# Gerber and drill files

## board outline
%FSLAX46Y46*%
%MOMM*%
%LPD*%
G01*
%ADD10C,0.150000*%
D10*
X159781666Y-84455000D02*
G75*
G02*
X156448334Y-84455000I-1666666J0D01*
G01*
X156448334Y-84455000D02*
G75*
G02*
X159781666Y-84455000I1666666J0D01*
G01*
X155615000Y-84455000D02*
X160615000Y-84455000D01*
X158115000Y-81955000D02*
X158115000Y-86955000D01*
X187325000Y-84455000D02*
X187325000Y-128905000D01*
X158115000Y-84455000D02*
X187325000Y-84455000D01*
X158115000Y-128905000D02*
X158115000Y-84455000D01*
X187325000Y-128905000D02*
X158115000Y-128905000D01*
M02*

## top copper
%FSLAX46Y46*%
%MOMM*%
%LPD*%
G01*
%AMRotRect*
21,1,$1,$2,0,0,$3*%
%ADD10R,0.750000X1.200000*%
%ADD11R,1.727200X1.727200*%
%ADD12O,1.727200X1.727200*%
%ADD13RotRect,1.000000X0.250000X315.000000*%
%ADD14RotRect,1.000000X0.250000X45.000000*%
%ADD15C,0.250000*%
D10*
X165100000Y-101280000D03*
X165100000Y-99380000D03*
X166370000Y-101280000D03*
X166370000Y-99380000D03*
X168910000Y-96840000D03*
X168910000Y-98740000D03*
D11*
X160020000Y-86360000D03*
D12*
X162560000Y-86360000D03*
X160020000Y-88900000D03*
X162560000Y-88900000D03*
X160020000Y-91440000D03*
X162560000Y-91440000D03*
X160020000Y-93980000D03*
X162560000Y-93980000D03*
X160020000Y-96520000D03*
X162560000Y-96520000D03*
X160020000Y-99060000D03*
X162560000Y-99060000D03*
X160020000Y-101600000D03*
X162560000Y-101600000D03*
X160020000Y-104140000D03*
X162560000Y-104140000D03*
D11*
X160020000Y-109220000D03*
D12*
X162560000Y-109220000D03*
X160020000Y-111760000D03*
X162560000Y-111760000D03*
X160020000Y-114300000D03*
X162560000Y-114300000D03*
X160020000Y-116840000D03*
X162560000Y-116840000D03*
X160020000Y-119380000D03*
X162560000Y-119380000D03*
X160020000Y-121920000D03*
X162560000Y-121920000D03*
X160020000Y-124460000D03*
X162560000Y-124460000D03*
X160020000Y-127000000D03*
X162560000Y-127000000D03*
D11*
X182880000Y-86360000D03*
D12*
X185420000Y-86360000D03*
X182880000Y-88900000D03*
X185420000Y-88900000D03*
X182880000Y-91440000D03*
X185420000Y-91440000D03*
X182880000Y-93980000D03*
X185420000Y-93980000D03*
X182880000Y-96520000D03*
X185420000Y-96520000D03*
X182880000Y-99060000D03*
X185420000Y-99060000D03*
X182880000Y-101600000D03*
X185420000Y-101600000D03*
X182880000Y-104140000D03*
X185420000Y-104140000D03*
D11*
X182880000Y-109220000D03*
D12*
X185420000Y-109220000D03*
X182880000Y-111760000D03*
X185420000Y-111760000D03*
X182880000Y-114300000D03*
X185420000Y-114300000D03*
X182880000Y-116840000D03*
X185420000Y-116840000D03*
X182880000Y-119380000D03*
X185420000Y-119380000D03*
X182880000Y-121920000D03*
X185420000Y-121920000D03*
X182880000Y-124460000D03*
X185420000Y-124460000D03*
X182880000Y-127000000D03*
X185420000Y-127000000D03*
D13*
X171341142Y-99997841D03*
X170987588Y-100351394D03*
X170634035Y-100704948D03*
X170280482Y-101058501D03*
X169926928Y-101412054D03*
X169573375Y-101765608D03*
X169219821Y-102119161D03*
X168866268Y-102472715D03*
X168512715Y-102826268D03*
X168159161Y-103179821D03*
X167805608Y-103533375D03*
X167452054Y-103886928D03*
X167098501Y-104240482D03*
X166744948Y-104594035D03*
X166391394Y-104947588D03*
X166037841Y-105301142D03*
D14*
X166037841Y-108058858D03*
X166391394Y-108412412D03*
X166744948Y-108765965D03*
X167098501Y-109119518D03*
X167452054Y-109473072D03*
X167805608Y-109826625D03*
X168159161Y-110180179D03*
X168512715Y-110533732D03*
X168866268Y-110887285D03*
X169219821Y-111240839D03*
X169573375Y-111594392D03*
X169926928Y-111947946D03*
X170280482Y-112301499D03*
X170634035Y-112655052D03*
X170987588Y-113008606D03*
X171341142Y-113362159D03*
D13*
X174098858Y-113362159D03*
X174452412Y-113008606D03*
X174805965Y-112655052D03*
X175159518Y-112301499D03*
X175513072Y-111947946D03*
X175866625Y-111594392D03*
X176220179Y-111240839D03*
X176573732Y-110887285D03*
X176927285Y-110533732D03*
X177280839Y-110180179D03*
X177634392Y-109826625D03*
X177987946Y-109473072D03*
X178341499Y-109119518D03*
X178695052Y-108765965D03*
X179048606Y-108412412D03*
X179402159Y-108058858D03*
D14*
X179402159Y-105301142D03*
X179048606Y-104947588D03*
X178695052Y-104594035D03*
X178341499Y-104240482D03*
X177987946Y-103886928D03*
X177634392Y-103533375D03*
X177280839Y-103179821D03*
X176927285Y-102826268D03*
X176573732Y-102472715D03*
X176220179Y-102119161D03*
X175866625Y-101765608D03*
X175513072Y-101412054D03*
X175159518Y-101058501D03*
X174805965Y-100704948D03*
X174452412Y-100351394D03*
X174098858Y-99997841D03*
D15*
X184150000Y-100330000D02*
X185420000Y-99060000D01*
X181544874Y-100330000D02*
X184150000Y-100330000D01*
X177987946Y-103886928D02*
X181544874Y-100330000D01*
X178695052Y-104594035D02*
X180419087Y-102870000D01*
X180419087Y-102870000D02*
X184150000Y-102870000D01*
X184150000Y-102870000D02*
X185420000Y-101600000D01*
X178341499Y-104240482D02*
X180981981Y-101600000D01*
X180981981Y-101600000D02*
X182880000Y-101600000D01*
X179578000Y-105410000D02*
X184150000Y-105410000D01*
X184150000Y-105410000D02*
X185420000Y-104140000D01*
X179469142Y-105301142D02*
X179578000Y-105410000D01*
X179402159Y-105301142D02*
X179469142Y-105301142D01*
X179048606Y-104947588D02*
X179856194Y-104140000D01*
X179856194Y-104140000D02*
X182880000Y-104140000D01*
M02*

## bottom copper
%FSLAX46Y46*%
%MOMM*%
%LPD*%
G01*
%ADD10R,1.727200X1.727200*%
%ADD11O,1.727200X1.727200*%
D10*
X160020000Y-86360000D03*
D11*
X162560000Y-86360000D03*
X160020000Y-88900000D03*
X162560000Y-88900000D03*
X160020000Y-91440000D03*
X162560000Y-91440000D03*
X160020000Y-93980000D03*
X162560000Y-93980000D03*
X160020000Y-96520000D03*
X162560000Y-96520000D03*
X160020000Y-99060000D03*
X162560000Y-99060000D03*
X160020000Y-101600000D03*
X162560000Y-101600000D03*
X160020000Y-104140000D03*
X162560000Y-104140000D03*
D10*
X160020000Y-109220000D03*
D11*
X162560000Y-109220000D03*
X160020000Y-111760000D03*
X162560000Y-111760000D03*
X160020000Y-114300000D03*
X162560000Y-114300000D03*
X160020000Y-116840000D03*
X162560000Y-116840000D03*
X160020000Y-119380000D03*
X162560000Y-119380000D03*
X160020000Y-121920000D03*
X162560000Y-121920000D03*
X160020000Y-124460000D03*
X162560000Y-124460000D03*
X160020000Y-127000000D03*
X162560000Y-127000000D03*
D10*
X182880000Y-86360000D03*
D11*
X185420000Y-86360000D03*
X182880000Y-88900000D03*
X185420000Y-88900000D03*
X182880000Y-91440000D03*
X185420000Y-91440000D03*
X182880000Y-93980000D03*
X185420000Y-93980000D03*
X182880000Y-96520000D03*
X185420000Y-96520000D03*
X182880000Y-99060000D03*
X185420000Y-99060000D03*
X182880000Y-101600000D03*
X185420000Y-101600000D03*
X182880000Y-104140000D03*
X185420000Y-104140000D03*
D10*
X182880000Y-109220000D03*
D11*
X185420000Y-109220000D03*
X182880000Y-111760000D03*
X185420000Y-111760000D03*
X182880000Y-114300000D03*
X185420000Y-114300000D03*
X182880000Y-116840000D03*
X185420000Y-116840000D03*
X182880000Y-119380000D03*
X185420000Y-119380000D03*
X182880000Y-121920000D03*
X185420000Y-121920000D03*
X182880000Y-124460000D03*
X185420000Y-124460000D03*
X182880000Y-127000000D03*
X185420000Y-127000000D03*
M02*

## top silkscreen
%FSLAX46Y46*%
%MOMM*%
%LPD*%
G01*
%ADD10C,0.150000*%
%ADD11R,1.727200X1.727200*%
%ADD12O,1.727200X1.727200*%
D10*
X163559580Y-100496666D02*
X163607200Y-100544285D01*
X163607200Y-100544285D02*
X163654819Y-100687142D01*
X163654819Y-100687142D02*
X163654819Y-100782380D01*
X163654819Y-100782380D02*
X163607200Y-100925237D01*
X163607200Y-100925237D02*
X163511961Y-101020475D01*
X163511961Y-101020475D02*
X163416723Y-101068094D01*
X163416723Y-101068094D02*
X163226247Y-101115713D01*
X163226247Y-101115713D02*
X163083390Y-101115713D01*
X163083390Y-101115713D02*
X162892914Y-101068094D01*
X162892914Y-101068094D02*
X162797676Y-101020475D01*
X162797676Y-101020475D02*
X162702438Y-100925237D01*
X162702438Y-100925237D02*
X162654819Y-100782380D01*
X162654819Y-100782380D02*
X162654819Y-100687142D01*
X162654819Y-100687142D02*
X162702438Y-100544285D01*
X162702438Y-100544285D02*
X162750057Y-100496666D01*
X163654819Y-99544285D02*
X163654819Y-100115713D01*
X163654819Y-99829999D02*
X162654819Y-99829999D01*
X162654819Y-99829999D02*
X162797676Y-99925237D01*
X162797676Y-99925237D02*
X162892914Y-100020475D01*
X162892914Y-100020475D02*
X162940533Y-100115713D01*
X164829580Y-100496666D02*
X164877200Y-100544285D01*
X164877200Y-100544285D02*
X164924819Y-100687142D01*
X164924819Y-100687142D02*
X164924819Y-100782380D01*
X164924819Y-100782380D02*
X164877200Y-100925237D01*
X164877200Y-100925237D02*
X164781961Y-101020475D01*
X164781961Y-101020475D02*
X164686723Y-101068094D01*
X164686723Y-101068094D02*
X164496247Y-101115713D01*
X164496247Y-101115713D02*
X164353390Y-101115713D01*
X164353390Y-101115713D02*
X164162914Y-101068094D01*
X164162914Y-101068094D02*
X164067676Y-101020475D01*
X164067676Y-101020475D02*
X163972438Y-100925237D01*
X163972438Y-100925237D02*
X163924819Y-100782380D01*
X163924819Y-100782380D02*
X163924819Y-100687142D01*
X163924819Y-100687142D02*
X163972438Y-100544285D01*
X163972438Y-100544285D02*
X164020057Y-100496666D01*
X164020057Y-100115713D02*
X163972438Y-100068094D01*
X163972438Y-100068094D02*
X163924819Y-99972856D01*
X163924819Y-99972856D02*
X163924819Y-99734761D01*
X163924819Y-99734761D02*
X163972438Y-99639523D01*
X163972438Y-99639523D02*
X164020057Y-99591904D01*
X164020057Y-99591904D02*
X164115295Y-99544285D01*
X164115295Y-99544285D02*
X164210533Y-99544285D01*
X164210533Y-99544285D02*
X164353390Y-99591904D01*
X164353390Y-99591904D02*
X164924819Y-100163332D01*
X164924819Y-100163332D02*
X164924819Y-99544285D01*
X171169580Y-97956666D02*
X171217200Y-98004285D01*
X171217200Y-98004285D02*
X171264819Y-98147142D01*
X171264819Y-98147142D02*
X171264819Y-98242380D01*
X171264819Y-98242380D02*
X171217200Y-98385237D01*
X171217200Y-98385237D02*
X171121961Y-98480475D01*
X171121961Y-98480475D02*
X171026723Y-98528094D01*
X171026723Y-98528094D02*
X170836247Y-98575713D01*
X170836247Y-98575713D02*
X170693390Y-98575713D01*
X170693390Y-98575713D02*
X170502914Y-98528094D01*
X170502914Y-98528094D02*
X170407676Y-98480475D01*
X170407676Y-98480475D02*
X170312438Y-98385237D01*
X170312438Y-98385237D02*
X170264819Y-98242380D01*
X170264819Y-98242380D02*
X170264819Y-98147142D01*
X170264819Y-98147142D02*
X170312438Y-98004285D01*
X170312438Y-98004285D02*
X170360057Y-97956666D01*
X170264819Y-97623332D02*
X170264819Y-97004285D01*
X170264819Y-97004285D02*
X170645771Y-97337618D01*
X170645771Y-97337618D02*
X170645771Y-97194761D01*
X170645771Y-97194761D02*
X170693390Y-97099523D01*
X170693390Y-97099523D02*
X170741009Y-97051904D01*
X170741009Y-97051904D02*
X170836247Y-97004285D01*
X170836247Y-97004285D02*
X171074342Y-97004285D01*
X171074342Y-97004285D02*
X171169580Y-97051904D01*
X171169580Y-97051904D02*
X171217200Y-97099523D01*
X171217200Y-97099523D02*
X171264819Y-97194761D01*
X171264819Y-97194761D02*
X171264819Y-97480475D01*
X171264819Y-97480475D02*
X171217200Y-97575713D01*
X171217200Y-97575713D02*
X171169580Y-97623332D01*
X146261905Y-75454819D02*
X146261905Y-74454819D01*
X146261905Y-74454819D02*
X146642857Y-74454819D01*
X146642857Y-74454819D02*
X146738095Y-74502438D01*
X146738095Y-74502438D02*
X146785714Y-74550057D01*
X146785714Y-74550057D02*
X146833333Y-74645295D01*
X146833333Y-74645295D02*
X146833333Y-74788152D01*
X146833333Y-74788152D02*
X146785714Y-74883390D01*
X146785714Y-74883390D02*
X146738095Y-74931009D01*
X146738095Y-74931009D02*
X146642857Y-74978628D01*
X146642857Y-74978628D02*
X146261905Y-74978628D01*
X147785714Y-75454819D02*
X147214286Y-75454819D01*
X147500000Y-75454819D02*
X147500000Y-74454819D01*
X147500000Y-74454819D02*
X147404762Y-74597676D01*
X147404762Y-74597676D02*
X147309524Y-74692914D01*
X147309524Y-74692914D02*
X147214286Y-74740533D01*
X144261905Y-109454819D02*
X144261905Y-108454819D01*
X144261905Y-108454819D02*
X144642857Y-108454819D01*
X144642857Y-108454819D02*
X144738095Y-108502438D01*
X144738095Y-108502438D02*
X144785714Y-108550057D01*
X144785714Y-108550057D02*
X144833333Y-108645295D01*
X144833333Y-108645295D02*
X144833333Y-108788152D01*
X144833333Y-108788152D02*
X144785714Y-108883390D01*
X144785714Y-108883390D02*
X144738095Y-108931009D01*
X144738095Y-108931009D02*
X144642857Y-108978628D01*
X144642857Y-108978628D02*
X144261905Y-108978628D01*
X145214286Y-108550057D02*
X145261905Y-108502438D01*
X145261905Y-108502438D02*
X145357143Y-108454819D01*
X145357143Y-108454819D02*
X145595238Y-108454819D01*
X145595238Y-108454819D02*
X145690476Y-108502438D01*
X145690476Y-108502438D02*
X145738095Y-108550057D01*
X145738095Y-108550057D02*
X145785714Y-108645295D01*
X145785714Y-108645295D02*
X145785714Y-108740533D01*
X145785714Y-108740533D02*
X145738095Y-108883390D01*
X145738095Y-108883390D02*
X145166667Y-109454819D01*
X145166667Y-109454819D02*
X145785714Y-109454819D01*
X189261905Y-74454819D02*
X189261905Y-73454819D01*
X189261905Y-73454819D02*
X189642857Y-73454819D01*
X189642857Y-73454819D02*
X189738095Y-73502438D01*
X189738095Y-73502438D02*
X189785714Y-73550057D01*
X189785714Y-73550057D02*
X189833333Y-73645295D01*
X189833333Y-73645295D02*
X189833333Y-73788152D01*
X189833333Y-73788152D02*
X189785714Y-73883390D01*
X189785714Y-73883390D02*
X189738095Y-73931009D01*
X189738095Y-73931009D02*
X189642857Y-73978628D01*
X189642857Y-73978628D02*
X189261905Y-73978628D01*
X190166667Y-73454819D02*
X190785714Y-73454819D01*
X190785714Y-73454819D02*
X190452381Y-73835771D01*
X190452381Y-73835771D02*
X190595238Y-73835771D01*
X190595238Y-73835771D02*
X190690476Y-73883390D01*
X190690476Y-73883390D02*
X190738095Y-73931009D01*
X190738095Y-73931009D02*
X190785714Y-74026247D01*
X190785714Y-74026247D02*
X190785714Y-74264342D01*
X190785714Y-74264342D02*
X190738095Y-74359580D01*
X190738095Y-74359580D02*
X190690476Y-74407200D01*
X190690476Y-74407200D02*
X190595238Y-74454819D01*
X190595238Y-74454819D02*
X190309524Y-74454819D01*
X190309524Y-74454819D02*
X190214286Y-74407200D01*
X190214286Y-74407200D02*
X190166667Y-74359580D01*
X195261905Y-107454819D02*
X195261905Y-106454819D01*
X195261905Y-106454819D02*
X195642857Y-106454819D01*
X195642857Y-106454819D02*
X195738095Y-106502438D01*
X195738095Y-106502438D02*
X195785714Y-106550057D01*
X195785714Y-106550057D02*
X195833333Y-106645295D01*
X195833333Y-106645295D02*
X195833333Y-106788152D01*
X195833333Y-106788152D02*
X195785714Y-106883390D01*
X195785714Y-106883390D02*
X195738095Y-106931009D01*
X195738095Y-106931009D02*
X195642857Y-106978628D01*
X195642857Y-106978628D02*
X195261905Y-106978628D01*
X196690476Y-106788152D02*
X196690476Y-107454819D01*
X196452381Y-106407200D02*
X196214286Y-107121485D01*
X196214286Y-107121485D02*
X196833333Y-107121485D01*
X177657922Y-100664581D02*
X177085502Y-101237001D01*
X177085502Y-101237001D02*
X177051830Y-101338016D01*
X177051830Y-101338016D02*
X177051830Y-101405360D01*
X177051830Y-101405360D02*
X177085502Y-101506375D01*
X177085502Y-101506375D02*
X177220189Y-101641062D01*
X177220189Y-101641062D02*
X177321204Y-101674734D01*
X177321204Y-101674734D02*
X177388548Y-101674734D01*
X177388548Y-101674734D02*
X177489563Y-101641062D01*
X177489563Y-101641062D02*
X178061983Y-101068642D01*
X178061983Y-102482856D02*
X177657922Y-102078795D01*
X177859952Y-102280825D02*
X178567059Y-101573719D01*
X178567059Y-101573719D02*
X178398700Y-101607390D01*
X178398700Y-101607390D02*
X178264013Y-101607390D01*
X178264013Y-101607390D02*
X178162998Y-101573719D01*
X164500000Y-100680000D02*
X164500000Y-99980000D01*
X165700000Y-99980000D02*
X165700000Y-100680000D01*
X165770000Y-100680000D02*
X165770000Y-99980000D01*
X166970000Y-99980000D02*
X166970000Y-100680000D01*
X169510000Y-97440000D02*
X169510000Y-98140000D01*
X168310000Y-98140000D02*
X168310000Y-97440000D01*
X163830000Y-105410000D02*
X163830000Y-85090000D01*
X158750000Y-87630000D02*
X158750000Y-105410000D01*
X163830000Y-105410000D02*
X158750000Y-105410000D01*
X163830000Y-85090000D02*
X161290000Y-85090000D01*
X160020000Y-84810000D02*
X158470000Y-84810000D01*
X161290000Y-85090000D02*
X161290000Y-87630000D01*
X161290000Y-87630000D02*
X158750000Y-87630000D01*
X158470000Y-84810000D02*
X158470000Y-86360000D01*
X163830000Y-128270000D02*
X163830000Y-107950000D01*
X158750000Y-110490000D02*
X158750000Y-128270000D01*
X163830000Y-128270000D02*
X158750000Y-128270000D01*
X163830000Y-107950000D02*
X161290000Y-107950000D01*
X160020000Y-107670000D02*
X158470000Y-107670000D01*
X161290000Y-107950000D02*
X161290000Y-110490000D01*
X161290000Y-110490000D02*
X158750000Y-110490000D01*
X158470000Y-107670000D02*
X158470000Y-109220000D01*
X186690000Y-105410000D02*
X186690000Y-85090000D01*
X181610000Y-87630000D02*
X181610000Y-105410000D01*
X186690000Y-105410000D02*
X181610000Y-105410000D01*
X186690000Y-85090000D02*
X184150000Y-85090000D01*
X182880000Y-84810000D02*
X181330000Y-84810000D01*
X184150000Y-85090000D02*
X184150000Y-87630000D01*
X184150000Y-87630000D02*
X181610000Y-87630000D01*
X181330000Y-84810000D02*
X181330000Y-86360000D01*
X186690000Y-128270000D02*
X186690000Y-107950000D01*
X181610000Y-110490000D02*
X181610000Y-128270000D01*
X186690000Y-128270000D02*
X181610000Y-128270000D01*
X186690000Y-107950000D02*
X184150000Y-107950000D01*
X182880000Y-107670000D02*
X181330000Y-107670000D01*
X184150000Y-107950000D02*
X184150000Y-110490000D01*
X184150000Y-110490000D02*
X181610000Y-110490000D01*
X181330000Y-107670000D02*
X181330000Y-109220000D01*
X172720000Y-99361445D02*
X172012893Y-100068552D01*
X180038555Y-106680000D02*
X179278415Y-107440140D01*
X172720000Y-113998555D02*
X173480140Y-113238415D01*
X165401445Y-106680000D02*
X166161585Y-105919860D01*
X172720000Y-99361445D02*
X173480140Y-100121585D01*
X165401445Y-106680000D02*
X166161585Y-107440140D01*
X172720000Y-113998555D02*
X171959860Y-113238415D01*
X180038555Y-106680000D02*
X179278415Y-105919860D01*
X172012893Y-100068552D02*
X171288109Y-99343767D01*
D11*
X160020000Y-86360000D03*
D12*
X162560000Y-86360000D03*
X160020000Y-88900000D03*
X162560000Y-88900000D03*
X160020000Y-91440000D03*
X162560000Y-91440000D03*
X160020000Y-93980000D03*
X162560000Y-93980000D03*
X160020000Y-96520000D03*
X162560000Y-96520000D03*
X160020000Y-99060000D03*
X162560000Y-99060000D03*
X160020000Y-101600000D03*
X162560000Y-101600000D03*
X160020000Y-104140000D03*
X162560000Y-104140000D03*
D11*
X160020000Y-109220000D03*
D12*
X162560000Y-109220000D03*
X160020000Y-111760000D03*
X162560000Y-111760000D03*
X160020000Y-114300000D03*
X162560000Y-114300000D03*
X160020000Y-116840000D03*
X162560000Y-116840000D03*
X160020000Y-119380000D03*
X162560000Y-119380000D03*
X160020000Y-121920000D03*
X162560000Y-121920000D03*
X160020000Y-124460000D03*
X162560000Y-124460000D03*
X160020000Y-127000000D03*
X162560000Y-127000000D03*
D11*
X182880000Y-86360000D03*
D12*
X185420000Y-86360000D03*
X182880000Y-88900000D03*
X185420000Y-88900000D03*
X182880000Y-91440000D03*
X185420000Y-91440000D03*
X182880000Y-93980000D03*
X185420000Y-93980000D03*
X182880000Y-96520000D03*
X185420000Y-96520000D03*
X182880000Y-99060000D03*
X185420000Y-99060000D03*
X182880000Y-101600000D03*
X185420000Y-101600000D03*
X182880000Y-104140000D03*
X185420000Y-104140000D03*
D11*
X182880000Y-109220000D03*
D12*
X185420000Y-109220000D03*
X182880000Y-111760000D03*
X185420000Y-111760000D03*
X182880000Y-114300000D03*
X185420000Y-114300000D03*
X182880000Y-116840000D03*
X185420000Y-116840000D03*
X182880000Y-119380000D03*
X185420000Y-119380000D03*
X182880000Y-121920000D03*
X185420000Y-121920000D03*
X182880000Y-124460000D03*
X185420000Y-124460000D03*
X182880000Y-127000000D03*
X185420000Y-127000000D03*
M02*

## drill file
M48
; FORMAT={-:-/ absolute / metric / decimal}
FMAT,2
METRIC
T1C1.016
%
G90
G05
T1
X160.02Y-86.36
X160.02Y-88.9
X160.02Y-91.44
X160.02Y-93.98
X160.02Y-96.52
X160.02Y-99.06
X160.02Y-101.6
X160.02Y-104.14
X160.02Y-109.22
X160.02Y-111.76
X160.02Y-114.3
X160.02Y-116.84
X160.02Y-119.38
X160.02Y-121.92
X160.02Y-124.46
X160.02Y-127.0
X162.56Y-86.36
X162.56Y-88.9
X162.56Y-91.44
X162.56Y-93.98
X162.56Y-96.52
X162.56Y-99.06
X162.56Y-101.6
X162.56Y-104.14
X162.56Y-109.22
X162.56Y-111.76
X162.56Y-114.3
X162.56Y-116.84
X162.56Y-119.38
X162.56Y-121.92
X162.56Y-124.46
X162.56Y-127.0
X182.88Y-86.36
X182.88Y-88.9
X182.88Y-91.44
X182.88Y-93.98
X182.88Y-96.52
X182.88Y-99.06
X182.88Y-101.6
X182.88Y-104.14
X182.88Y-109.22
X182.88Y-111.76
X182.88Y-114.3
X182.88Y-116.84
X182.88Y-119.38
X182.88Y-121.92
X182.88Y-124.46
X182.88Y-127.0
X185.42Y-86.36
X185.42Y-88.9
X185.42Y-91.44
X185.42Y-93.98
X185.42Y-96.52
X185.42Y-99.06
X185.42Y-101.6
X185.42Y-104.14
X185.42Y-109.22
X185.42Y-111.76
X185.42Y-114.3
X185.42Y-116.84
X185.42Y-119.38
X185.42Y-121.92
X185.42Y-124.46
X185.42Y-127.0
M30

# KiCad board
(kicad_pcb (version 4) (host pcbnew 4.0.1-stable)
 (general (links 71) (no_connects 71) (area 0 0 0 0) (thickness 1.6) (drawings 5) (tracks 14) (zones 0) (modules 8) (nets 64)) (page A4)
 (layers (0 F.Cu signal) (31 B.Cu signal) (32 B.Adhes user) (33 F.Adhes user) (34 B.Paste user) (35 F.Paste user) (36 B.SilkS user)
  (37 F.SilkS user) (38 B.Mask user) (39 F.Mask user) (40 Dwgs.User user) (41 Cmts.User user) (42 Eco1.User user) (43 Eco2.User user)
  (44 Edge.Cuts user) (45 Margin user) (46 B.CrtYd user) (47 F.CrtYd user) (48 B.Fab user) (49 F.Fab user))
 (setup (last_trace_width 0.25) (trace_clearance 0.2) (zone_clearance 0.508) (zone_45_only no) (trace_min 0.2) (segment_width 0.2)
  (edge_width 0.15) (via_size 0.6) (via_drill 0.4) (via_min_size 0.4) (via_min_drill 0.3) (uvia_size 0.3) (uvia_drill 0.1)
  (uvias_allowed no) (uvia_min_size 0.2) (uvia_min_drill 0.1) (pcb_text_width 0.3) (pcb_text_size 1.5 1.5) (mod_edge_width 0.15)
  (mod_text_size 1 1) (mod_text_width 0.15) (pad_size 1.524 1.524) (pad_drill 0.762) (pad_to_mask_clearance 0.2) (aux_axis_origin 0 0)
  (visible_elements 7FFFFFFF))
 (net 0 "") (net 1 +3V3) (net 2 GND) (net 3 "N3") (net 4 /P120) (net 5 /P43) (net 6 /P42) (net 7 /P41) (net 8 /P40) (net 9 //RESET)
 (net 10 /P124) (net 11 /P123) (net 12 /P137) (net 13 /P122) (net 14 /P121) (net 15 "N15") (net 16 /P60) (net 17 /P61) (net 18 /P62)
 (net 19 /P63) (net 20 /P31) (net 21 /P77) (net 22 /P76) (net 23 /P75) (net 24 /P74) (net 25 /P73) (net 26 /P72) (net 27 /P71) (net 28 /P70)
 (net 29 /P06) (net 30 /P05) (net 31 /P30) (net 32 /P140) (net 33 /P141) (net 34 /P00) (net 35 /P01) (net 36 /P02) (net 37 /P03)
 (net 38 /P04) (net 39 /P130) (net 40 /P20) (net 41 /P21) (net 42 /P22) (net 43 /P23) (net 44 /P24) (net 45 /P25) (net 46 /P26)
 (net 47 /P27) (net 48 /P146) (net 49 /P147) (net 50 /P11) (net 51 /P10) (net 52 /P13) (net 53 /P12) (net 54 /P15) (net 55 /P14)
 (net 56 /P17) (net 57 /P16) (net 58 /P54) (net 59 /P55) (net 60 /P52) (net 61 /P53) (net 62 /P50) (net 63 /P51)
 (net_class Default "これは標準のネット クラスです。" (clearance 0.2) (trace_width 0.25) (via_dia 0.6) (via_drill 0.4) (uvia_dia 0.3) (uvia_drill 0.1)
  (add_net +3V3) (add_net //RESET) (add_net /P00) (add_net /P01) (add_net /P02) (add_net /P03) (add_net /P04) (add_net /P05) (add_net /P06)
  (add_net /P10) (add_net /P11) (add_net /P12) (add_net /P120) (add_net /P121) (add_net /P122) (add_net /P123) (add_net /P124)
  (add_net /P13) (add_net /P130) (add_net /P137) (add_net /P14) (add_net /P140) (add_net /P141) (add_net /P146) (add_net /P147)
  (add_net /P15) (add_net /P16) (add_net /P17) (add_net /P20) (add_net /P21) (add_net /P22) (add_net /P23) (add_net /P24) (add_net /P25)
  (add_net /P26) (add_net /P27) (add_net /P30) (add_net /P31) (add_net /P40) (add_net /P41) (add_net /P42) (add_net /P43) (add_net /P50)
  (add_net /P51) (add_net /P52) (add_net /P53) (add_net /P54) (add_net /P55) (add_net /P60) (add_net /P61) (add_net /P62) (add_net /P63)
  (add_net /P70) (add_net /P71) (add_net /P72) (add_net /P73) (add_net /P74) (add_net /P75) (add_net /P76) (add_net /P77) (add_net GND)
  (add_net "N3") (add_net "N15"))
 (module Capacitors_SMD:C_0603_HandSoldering (layer F.Cu) (at 165.1 100.33 90)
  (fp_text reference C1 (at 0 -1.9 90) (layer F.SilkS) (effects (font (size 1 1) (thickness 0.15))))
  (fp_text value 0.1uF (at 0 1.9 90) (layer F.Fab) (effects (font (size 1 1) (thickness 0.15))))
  (fp_line (start -0.35 -0.6) (end 0.35 -0.6) (layer F.SilkS) (width 0.15))
  (fp_line (start 0.35 0.6) (end -0.35 0.6) (layer F.SilkS) (width 0.15))
  (pad 1 smd rect (at -0.95 0 90) (size 1.2 0.75) (layers F.Cu F.Paste F.Mask) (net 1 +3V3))
  (pad 2 smd rect (at 0.95 0 90) (size 1.2 0.75) (layers F.Cu F.Paste F.Mask) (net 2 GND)))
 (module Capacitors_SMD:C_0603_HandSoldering (layer F.Cu) (at 166.37 100.33 90)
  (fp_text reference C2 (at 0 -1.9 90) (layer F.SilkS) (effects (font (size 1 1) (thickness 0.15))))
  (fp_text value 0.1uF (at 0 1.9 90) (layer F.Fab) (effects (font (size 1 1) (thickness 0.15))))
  (fp_line (start -0.35 -0.6) (end 0.35 -0.6) (layer F.SilkS) (width 0.15))
  (fp_line (start 0.35 0.6) (end -0.35 0.6) (layer F.SilkS) (width 0.15))
  (pad 1 smd rect (at -0.95 0 90) (size 1.2 0.75) (layers F.Cu F.Paste F.Mask) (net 1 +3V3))
  (pad 2 smd rect (at 0.95 0 90) (size 1.2 0.75) (layers F.Cu F.Paste F.Mask) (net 2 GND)))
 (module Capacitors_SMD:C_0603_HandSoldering (layer F.Cu) (at 168.91 97.79 270)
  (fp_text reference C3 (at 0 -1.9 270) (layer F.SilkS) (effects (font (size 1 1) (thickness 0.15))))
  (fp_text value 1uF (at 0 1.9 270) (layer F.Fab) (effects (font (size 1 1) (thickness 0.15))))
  (fp_line (start -0.35 -0.6) (end 0.35 -0.6) (layer F.SilkS) (width 0.15))
  (fp_line (start 0.35 0.6) (end -0.35 0.6) (layer F.SilkS) (width 0.15))
  (pad 1 smd rect (at -0.95 0 270) (size 1.2 0.75) (layers F.Cu F.Paste F.Mask) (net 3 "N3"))
  (pad 2 smd rect (at 0.95 0 270) (size 1.2 0.75) (layers F.Cu F.Paste F.Mask) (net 2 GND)))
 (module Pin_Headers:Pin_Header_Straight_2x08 (layer F.Cu) (at 160.02 86.36)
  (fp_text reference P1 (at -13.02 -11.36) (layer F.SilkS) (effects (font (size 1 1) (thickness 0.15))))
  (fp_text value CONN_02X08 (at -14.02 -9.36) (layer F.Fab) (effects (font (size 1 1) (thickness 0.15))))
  (fp_line (start 3.81 19.05) (end 3.81 -1.27) (layer F.SilkS) (width 0.15))
  (fp_line (start -1.27 1.27) (end -1.27 19.05) (layer F.SilkS) (width 0.15))
  (fp_line (start 3.81 19.05) (end -1.27 19.05) (layer F.SilkS) (width 0.15))
  (fp_line (start 3.81 -1.27) (end 1.27 -1.27) (layer F.SilkS) (width 0.15))
  (fp_line (start 0 -1.55) (end -1.55 -1.55) (layer F.SilkS) (width 0.15))
  (fp_line (start 1.27 -1.27) (end 1.27 1.27) (layer F.SilkS) (width 0.15))
  (fp_line (start 1.27 1.27) (end -1.27 1.27) (layer F.SilkS) (width 0.15))
  (fp_line (start -1.55 -1.55) (end -1.55 0) (layer F.SilkS) (width 0.15))
  (pad 1 thru_hole rect (at 0 0) (size 1.7272 1.7272) (drill 1.016) (layers *.Cu *.Mask F.SilkS) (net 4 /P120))
  (pad 2 thru_hole oval (at 2.54 0) (size 1.7272 1.7272) (drill 1.016) (layers *.Cu *.Mask F.SilkS) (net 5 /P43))
  (pad 3 thru_hole oval (at 0 2.54) (size 1.7272 1.7272) (drill 1.016) (layers *.Cu *.Mask F.SilkS) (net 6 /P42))
  (pad 4 thru_hole oval (at 2.54 2.54) (size 1.7272 1.7272) (drill 1.016) (layers *.Cu *.Mask F.SilkS) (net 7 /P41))
  (pad 5 thru_hole oval (at 0 5.08) (size 1.7272 1.7272) (drill 1.016) (layers *.Cu *.Mask F.SilkS) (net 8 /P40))
  (pad 6 thru_hole oval (at 2.54 5.08) (size 1.7272 1.7272) (drill 1.016) (layers *.Cu *.Mask F.SilkS) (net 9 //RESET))
  (pad 7 thru_hole oval (at 0 7.62) (size 1.7272 1.7272) (drill 1.016) (layers *.Cu *.Mask F.SilkS) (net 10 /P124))
  (pad 8 thru_hole oval (at 2.54 7.62) (size 1.7272 1.7272) (drill 1.016) (layers *.Cu *.Mask F.SilkS) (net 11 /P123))
  (pad 9 thru_hole oval (at 0 10.16) (size 1.7272 1.7272) (drill 1.016) (layers *.Cu *.Mask F.SilkS) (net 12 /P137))
  (pad 10 thru_hole oval (at 2.54 10.16) (size 1.7272 1.7272) (drill 1.016) (layers *.Cu *.Mask F.SilkS) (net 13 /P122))
  (pad 11 thru_hole oval (at 0 12.7) (size 1.7272 1.7272) (drill 1.016) (layers *.Cu *.Mask F.SilkS) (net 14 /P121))
  (pad 12 thru_hole oval (at 2.54 12.7) (size 1.7272 1.7272) (drill 1.016) (layers *.Cu *.Mask F.SilkS) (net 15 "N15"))
  (pad 13 thru_hole oval (at 0 15.24) (size 1.7272 1.7272) (drill 1.016) (layers *.Cu *.Mask F.SilkS) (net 2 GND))
  (pad 14 thru_hole oval (at 2.54 15.24) (size 1.7272 1.7272) (drill 1.016) (layers *.Cu *.Mask F.SilkS) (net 2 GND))
  (pad 15 thru_hole oval (at 0 17.78) (size 1.7272 1.7272) (drill 1.016) (layers *.Cu *.Mask F.SilkS) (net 1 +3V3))
  (pad 16 thru_hole oval (at 2.54 17.78) (size 1.7272 1.7272) (drill 1.016) (layers *.Cu *.Mask F.SilkS) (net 1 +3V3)))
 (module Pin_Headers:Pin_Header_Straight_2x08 (layer F.Cu) (at 160.02 109.22)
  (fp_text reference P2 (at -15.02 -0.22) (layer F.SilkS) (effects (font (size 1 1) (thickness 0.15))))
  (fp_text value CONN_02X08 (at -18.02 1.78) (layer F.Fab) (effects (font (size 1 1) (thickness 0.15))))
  (fp_line (start 3.81 19.05) (end 3.81 -1.27) (layer F.SilkS) (width 0.15))
  (fp_line (start -1.27 1.27) (end -1.27 19.05) (layer F.SilkS) (width 0.15))
  (fp_line (start 3.81 19.05) (end -1.27 19.05) (layer F.SilkS) (width 0.15))
  (fp_line (start 3.81 -1.27) (end 1.27 -1.27) (layer F.SilkS) (width 0.15))
  (fp_line (start 0 -1.55) (end -1.55 -1.55) (layer F.SilkS) (width 0.15))
  (fp_line (start 1.27 -1.27) (end 1.27 1.27) (layer F.SilkS) (width 0.15))
  (fp_line (start 1.27 1.27) (end -1.27 1.27) (layer F.SilkS) (width 0.15))
  (fp_line (start -1.55 -1.55) (end -1.55 0) (layer F.SilkS) (width 0.15))
  (pad 1 thru_hole rect (at 0 0) (size 1.7272 1.7272) (drill 1.016) (layers *.Cu *.Mask F.SilkS) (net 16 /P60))
  (pad 2 thru_hole oval (at 2.54 0) (size 1.7272 1.7272) (drill 1.016) (layers *.Cu *.Mask F.SilkS) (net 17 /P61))
  (pad 3 thru_hole oval (at 0 2.54) (size 1.7272 1.7272) (drill 1.016) (layers *.Cu *.Mask F.SilkS) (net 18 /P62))
  (pad 4 thru_hole oval (at 2.54 2.54) (size 1.7272 1.7272) (drill 1.016) (layers *.Cu *.Mask F.SilkS) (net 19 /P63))
  (pad 5 thru_hole oval (at 0 5.08) (size 1.7272 1.7272) (drill 1.016) (layers *.Cu *.Mask F.SilkS) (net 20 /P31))
  (pad 6 thru_hole oval (at 2.54 5.08) (size 1.7272 1.7272) (drill 1.016) (layers *.Cu *.Mask F.SilkS) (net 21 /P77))
  (pad 7 thru_hole oval (at 0 7.62) (size 1.7272 1.7272) (drill 1.016) (layers *.Cu *.Mask F.SilkS) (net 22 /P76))
  (pad 8 thru_hole oval (at 2.54 7.62) (size 1.7272 1.7272) (drill 1.016) (layers *.Cu *.Mask F.SilkS) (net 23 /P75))
  (pad 9 thru_hole oval (at 0 10.16) (size 1.7272 1.7272) (drill 1.016) (layers *.Cu *.Mask F.SilkS) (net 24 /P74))
  (pad 10 thru_hole oval (at 2.54 10.16) (size 1.7272 1.7272) (drill 1.016) (layers *.Cu *.Mask F.SilkS) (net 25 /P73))
  (pad 11 thru_hole oval (at 0 12.7) (size 1.7272 1.7272) (drill 1.016) (layers *.Cu *.Mask F.SilkS) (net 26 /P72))
  (pad 12 thru_hole oval (at 2.54 12.7) (size 1.7272 1.7272) (drill 1.016) (layers *.Cu *.Mask F.SilkS) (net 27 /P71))
  (pad 13 thru_hole oval (at 0 15.24) (size 1.7272 1.7272) (drill 1.016) (layers *.Cu *.Mask F.SilkS) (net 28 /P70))
  (pad 14 thru_hole oval (at 2.54 15.24) (size 1.7272 1.7272) (drill 1.016) (layers *.Cu *.Mask F.SilkS) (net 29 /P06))
  (pad 15 thru_hole oval (at 0 17.78) (size 1.7272 1.7272) (drill 1.016) (layers *.Cu *.Mask F.SilkS) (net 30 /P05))
  (pad 16 thru_hole oval (at 2.54 17.78) (size 1.7272 1.7272) (drill 1.016) (layers *.Cu *.Mask F.SilkS) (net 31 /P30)))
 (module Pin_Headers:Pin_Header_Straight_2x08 (layer F.Cu) (at 182.88 86.36)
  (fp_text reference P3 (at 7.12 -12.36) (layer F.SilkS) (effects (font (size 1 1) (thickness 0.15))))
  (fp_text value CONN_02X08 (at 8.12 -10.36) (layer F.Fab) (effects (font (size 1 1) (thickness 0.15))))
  (fp_line (start 3.81 19.05) (end 3.81 -1.27) (layer F.SilkS) (width 0.15))
  (fp_line (start -1.27 1.27) (end -1.27 19.05) (layer F.SilkS) (width 0.15))
  (fp_line (start 3.81 19.05) (end -1.27 19.05) (layer F.SilkS) (width 0.15))
  (fp_line (start 3.81 -1.27) (end 1.27 -1.27) (layer F.SilkS) (width 0.15))
  (fp_line (start 0 -1.55) (end -1.55 -1.55) (layer F.SilkS) (width 0.15))
  (fp_line (start 1.27 -1.27) (end 1.27 1.27) (layer F.SilkS) (width 0.15))
  (fp_line (start 1.27 1.27) (end -1.27 1.27) (layer F.SilkS) (width 0.15))
  (fp_line (start -1.55 -1.55) (end -1.55 0) (layer F.SilkS) (width 0.15))
  (pad 1 thru_hole rect (at 0 0) (size 1.7272 1.7272) (drill 1.016) (layers *.Cu *.Mask F.SilkS) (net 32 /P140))
  (pad 2 thru_hole oval (at 2.54 0) (size 1.7272 1.7272) (drill 1.016) (layers *.Cu *.Mask F.SilkS) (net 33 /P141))
  (pad 3 thru_hole oval (at 0 2.54) (size 1.7272 1.7272) (drill 1.016) (layers *.Cu *.Mask F.SilkS) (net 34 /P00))
  (pad 4 thru_hole oval (at 2.54 2.54) (size 1.7272 1.7272) (drill 1.016) (layers *.Cu *.Mask F.SilkS) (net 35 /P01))
  (pad 5 thru_hole oval (at 0 5.08) (size 1.7272 1.7272) (drill 1.016) (layers *.Cu *.Mask F.SilkS) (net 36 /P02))
  (pad 6 thru_hole oval (at 2.54 5.08) (size 1.7272 1.7272) (drill 1.016) (layers *.Cu *.Mask F.SilkS) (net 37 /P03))
  (pad 7 thru_hole oval (at 0 7.62) (size 1.7272 1.7272) (drill 1.016) (layers *.Cu *.Mask F.SilkS) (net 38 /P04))
  (pad 8 thru_hole oval (at 2.54 7.62) (size 1.7272 1.7272) (drill 1.016) (layers *.Cu *.Mask F.SilkS) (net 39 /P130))
  (pad 9 thru_hole oval (at 0 10.16) (size 1.7272 1.7272) (drill 1.016) (layers *.Cu *.Mask F.SilkS) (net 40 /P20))
  (pad 10 thru_hole oval (at 2.54 10.16) (size 1.7272 1.7272) (drill 1.016) (layers *.Cu *.Mask F.SilkS) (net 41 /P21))
  (pad 11 thru_hole oval (at 0 12.7) (size 1.7272 1.7272) (drill 1.016) (layers *.Cu *.Mask F.SilkS) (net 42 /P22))
  (pad 12 thru_hole oval (at 2.54 12.7) (size 1.7272 1.7272) (drill 1.016) (layers *.Cu *.Mask F.SilkS) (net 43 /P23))
  (pad 13 thru_hole oval (at 0 15.24) (size 1.7272 1.7272) (drill 1.016) (layers *.Cu *.Mask F.SilkS) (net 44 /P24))
  (pad 14 thru_hole oval (at 2.54 15.24) (size 1.7272 1.7272) (drill 1.016) (layers *.Cu *.Mask F.SilkS) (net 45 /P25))
  (pad 15 thru_hole oval (at 0 17.78) (size 1.7272 1.7272) (drill 1.016) (layers *.Cu *.Mask F.SilkS) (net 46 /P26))
  (pad 16 thru_hole oval (at 2.54 17.78) (size 1.7272 1.7272) (drill 1.016) (layers *.Cu *.Mask F.SilkS) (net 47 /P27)))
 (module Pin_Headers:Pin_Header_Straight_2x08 (layer F.Cu) (at 182.88 109.22)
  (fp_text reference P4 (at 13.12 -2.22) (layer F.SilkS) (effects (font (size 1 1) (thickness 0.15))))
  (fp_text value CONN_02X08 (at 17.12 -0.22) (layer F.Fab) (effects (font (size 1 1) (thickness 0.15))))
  (fp_line (start 3.81 19.05) (end 3.81 -1.27) (layer F.SilkS) (width 0.15))
  (fp_line (start -1.27 1.27) (end -1.27 19.05) (layer F.SilkS) (width 0.15))
  (fp_line (start 3.81 19.05) (end -1.27 19.05) (layer F.SilkS) (width 0.15))
  (fp_line (start 3.81 -1.27) (end 1.27 -1.27) (layer F.SilkS) (width 0.15))
  (fp_line (start 0 -1.55) (end -1.55 -1.55) (layer F.SilkS) (width 0.15))
  (fp_line (start 1.27 -1.27) (end 1.27 1.27) (layer F.SilkS) (width 0.15))
  (fp_line (start 1.27 1.27) (end -1.27 1.27) (layer F.SilkS) (width 0.15))
  (fp_line (start -1.55 -1.55) (end -1.55 0) (layer F.SilkS) (width 0.15))
  (pad 1 thru_hole rect (at 0 0) (size 1.7272 1.7272) (drill 1.016) (layers *.Cu *.Mask F.SilkS) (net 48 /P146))
  (pad 2 thru_hole oval (at 2.54 0) (size 1.7272 1.7272) (drill 1.016) (layers *.Cu *.Mask F.SilkS) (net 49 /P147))
  (pad 3 thru_hole oval (at 0 2.54) (size 1.7272 1.7272) (drill 1.016) (layers *.Cu *.Mask F.SilkS) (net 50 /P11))
  (pad 4 thru_hole oval (at 2.54 2.54) (size 1.7272 1.7272) (drill 1.016) (layers *.Cu *.Mask F.SilkS) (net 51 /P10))
  (pad 5 thru_hole oval (at 0 5.08) (size 1.7272 1.7272) (drill 1.016) (layers *.Cu *.Mask F.SilkS) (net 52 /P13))
  (pad 6 thru_hole oval (at 2.54 5.08) (size 1.7272 1.7272) (drill 1.016) (layers *.Cu *.Mask F.SilkS) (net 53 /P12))
  (pad 7 thru_hole oval (at 0 7.62) (size 1.7272 1.7272) (drill 1.016) (layers *.Cu *.Mask F.SilkS) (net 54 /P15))
  (pad 8 thru_hole oval (at 2.54 7.62) (size 1.7272 1.7272) (drill 1.016) (layers *.Cu *.Mask F.SilkS) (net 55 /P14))
  (pad 9 thru_hole oval (at 0 10.16) (size 1.7272 1.7272) (drill 1.016) (layers *.Cu *.Mask F.SilkS) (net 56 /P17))
  (pad 10 thru_hole oval (at 2.54 10.16) (size 1.7272 1.7272) (drill 1.016) (layers *.Cu *.Mask F.SilkS) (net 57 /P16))
  (pad 11 thru_hole oval (at 0 12.7) (size 1.7272 1.7272) (drill 1.016) (layers *.Cu *.Mask F.SilkS) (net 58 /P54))
  (pad 12 thru_hole oval (at 2.54 12.7) (size 1.7272 1.7272) (drill 1.016) (layers *.Cu *.Mask F.SilkS) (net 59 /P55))
  (pad 13 thru_hole oval (at 0 15.24) (size 1.7272 1.7272) (drill 1.016) (layers *.Cu *.Mask F.SilkS) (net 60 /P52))
  (pad 14 thru_hole oval (at 2.54 15.24) (size 1.7272 1.7272) (drill 1.016) (layers *.Cu *.Mask F.SilkS) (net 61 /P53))
  (pad 15 thru_hole oval (at 0 17.78) (size 1.7272 1.7272) (drill 1.016) (layers *.Cu *.Mask F.SilkS) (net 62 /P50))
  (pad 16 thru_hole oval (at 2.54 17.78) (size 1.7272 1.7272) (drill 1.016) (layers *.Cu *.Mask F.SilkS) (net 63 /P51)))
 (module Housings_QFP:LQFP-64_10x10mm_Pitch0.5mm (layer F.Cu) (at 172.72 106.68 315)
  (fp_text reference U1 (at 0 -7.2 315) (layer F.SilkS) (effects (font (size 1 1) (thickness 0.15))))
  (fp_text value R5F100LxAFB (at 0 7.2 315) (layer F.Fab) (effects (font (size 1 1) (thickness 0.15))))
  (fp_line (start -5.175 -5.175) (end -5.175 -4.175) (layer F.SilkS) (width 0.15))
  (fp_line (start 5.175 -5.175) (end 5.175 -4.1) (layer F.SilkS) (width 0.15))
  (fp_line (start 5.175 5.175) (end 5.175 4.1) (layer F.SilkS) (width 0.15))
  (fp_line (start -5.175 5.175) (end -5.175 4.1) (layer F.SilkS) (width 0.15))
  (fp_line (start -5.175 -5.175) (end -4.1 -5.175) (layer F.SilkS) (width 0.15))
  (fp_line (start -5.175 5.175) (end -4.1 5.175) (layer F.SilkS) (width 0.15))
  (fp_line (start 5.175 5.175) (end 4.1 5.175) (layer F.SilkS) (width 0.15))
  (fp_line (start 5.175 -5.175) (end 4.1 -5.175) (layer F.SilkS) (width 0.15))
  (fp_line (start -5.175 -4.175) (end -6.2 -4.175) (layer F.SilkS) (width 0.15))
  (pad 1 smd rect (at -5.7 -3.75 315) (size 1 0.25) (layers F.Cu F.Paste F.Mask) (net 4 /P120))
  (pad 2 smd rect (at -5.7 -3.25 315) (size 1 0.25) (layers F.Cu F.Paste F.Mask) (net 5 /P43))
  (pad 3 smd rect (at -5.7 -2.75 315) (size 1 0.25) (layers F.Cu F.Paste F.Mask) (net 6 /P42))
  (pad 4 smd rect (at -5.7 -2.25 315) (size 1 0.25) (layers F.Cu F.Paste F.Mask) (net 7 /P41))
  (pad 5 smd rect (at -5.7 -1.75 315) (size 1 0.25) (layers F.Cu F.Paste F.Mask) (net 8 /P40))
  (pad 6 smd rect (at -5.7 -1.25 315) (size 1 0.25) (layers F.Cu F.Paste F.Mask) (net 9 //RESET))
  (pad 7 smd rect (at -5.7 -0.75 315) (size 1 0.25) (layers F.Cu F.Paste F.Mask) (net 10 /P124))
  (pad 8 smd rect (at -5.7 -0.25 315) (size 1 0.25) (layers F.Cu F.Paste F.Mask) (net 11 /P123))
  (pad 9 smd rect (at -5.7 0.25 315) (size 1 0.25) (layers F.Cu F.Paste F.Mask) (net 12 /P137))
  (pad 10 smd rect (at -5.7 0.75 315) (size 1 0.25) (layers F.Cu F.Paste F.Mask) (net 13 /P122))
  (pad 11 smd rect (at -5.7 1.25 315) (size 1 0.25) (layers F.Cu F.Paste F.Mask) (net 14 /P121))
  (pad 12 smd rect (at -5.7 1.75 315) (size 1 0.25) (layers F.Cu F.Paste F.Mask) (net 3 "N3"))
  (pad 13 smd rect (at -5.7 2.25 315) (size 1 0.25) (layers F.Cu F.Paste F.Mask) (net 2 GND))
  (pad 14 smd rect (at -5.7 2.75 315) (size 1 0.25) (layers F.Cu F.Paste F.Mask) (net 2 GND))
  (pad 15 smd rect (at -5.7 3.25 315) (size 1 0.25) (layers F.Cu F.Paste F.Mask) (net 1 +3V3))
  (pad 16 smd rect (at -5.7 3.75 315) (size 1 0.25) (layers F.Cu F.Paste F.Mask) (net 1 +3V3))
  (pad 17 smd rect (at -3.75 5.7 45) (size 1 0.25) (layers F.Cu F.Paste F.Mask) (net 16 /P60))
  (pad 18 smd rect (at -3.25 5.7 45) (size 1 0.25) (layers F.Cu F.Paste F.Mask) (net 17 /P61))
  (pad 19 smd rect (at -2.75 5.7 45) (size 1 0.25) (layers F.Cu F.Paste F.Mask) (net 18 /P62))
  (pad 20 smd rect (at -2.25 5.7 45) (size 1 0.25) (layers F.Cu F.Paste F.Mask) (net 19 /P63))
  (pad 21 smd rect (at -1.75 5.7 45) (size 1 0.25) (layers F.Cu F.Paste F.Mask) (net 20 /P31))
  (pad 22 smd rect (at -1.25 5.7 45) (size 1 0.25) (layers F.Cu F.Paste F.Mask) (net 21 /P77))
  (pad 23 smd rect (at -0.75 5.7 45) (size 1 0.25) (layers F.Cu F.Paste F.Mask) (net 22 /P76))
  (pad 24 smd rect (at -0.25 5.7 45) (size 1 0.25) (layers F.Cu F.Paste F.Mask) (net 23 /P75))
  (pad 25 smd rect (at 0.25 5.7 45) (size 1 0.25) (layers F.Cu F.Paste F.Mask) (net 24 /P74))
  (pad 26 smd rect (at 0.75 5.7 45) (size 1 0.25) (layers F.Cu F.Paste F.Mask) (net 25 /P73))
  (pad 27 smd rect (at 1.25 5.7 45) (size 1 0.25) (layers F.Cu F.Paste F.Mask) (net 26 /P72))
  (pad 28 smd rect (at 1.75 5.7 45) (size 1 0.25) (layers F.Cu F.Paste F.Mask) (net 27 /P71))
  (pad 29 smd rect (at 2.25 5.7 45) (size 1 0.25) (layers F.Cu F.Paste F.Mask) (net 28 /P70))
  (pad 30 smd rect (at 2.75 5.7 45) (size 1 0.25) (layers F.Cu F.Paste F.Mask) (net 29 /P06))
  (pad 31 smd rect (at 3.25 5.7 45) (size 1 0.25) (layers F.Cu F.Paste F.Mask) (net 30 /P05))
  (pad 32 smd rect (at 3.75 5.7 45) (size 1 0.25) (layers F.Cu F.Paste F.Mask) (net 31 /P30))
  (pad 33 smd rect (at 5.7 3.75 315) (size 1 0.25) (layers F.Cu F.Paste F.Mask) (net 62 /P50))
  (pad 34 smd rect (at 5.7 3.25 315) (size 1 0.25) (layers F.Cu F.Paste F.Mask) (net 63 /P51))
  (pad 35 smd rect (at 5.7 2.75 315) (size 1 0.25) (layers F.Cu F.Paste F.Mask) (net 60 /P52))
  (pad 36 smd rect (at 5.7 2.25 315) (size 1 0.25) (layers F.Cu F.Paste F.Mask) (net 61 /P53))
  (pad 37 smd rect (at 5.7 1.75 315) (size 1 0.25) (layers F.Cu F.Paste F.Mask) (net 58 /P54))
  (pad 38 smd rect (at 5.7 1.25 315) (size 1 0.25) (layers F.Cu F.Paste F.Mask) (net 59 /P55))
  (pad 39 smd rect (at 5.7 0.75 315) (size 1 0.25) (layers F.Cu F.Paste F.Mask) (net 56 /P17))
  (pad 40 smd rect (at 5.7 0.25 315) (size 1 0.25) (layers F.Cu F.Paste F.Mask) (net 57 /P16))
  (pad 41 smd rect (at 5.7 -0.25 315) (size 1 0.25) (layers F.Cu F.Paste F.Mask) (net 54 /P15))
  (pad 42 smd rect (at 5.7 -0.75 315) (size 1 0.25) (layers F.Cu F.Paste F.Mask) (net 55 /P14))
  (pad 43 smd rect (at 5.7 -1.25 315) (size 1 0.25) (layers F.Cu F.Paste F.Mask) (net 52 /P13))
  (pad 44 smd rect (at 5.7 -1.75 315) (size 1 0.25) (layers F.Cu F.Paste F.Mask) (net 53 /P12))
  (pad 45 smd rect (at 5.7 -2.25 315) (size 1 0.25) (layers F.Cu F.Paste F.Mask) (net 50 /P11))
  (pad 46 smd rect (at 5.7 -2.75 315) (size 1 0.25) (layers F.Cu F.Paste F.Mask) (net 51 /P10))
  (pad 47 smd rect (at 5.7 -3.25 315) (size 1 0.25) (layers F.Cu F.Paste F.Mask) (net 48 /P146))
  (pad 48 smd rect (at 5.7 -3.75 315) (size 1 0.25) (layers F.Cu F.Paste F.Mask) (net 49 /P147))
  (pad 49 smd rect (at 3.75 -5.7 45) (size 1 0.25) (layers F.Cu F.Paste F.Mask) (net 47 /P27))
  (pad 50 smd rect (at 3.25 -5.7 45) (size 1 0.25) (layers F.Cu F.Paste F.Mask) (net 46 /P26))
  (pad 51 smd rect (at 2.75 -5.7 45) (size 1 0.25) (layers F.Cu F.Paste F.Mask) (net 45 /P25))
  (pad 52 smd rect (at 2.25 -5.7 45) (size 1 0.25) (layers F.Cu F.Paste F.Mask) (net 44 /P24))
  (pad 53 smd rect (at 1.75 -5.7 45) (size 1 0.25) (layers F.Cu F.Paste F.Mask) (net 43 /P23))
  (pad 54 smd rect (at 1.25 -5.7 45) (size 1 0.25) (layers F.Cu F.Paste F.Mask) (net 42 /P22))
  (pad 55 smd rect (at 0.75 -5.7 45) (size 1 0.25) (layers F.Cu F.Paste F.Mask) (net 41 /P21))
  (pad 56 smd rect (at 0.25 -5.7 45) (size 1 0.25) (layers F.Cu F.Paste F.Mask) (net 40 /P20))
  (pad 57 smd rect (at -0.25 -5.7 45) (size 1 0.25) (layers F.Cu F.Paste F.Mask) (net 39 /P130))
  (pad 58 smd rect (at -0.75 -5.7 45) (size 1 0.25) (layers F.Cu F.Paste F.Mask) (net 38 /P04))
  (pad 59 smd rect (at -1.25 -5.7 45) (size 1 0.25) (layers F.Cu F.Paste F.Mask) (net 37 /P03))
  (pad 60 smd rect (at -1.75 -5.7 45) (size 1 0.25) (layers F.Cu F.Paste F.Mask) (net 36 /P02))
  (pad 61 smd rect (at -2.25 -5.7 45) (size 1 0.25) (layers F.Cu F.Paste F.Mask) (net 35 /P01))
  (pad 62 smd rect (at -2.75 -5.7 45) (size 1 0.25) (layers F.Cu F.Paste F.Mask) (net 34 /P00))
  (pad 63 smd rect (at -3.25 -5.7 45) (size 1 0.25) (layers F.Cu F.Paste F.Mask) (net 33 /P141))
  (pad 64 smd rect (at -3.75 -5.7 45) (size 1 0.25) (layers F.Cu F.Paste F.Mask) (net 32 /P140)))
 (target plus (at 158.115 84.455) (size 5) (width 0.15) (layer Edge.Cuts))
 (gr_line (start 187.325 84.455) (end 187.325 128.905) (angle 90) (layer Edge.Cuts) (width 0.15))
 (gr_line (start 158.115 84.455) (end 187.325 84.455) (angle 90) (layer Edge.Cuts) (width 0.15))
 (gr_line (start 158.115 128.905) (end 158.115 84.455) (angle 90) (layer Edge.Cuts) (width 0.15))
 (gr_line (start 187.325 128.905) (end 158.115 128.905) (angle 90) (layer Edge.Cuts) (width 0.15))
 (segment (start 184.15 100.33) (end 185.42 99.06) (width 0.25) (layer F.Cu) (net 43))
 (segment (start 181.544874 100.33) (end 184.15 100.33) (width 0.25) (layer F.Cu) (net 43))
 (segment (start 177.987946 103.886928) (end 181.544874 100.33) (width 0.25) (layer F.Cu) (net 43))
 (segment (start 178.695052 104.594035) (end 180.419087 102.87) (width 0.25) (layer F.Cu) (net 45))
 (segment (start 180.419087 102.87) (end 184.15 102.87) (width 0.25) (layer F.Cu) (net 45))
 (segment (start 184.15 102.87) (end 185.42 101.6) (width 0.25) (layer F.Cu) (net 45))
 (segment (start 178.341499 104.240482) (end 180.981981 101.6) (width 0.25) (layer F.Cu) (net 44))
 (segment (start 180.981981 101.6) (end 182.88 101.6) (width 0.25) (layer F.Cu) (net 44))
 (segment (start 179.578 105.41) (end 184.15 105.41) (width 0.25) (layer F.Cu) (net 47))
 (segment (start 184.15 105.41) (end 185.42 104.14) (width 0.25) (layer F.Cu) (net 47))
 (segment (start 179.469142 105.301142) (end 179.578 105.41) (width 0.25) (layer F.Cu) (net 47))
 (segment (start 179.402159 105.301142) (end 179.469142 105.301142) (width 0.25) (layer F.Cu) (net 47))
 (segment (start 179.048606 104.947588) (end 179.856194 104.14) (width 0.25) (layer F.Cu) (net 46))
 (segment (start 179.856194 104.14) (end 182.88 104.14) (width 0.25) (layer F.Cu) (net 46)))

